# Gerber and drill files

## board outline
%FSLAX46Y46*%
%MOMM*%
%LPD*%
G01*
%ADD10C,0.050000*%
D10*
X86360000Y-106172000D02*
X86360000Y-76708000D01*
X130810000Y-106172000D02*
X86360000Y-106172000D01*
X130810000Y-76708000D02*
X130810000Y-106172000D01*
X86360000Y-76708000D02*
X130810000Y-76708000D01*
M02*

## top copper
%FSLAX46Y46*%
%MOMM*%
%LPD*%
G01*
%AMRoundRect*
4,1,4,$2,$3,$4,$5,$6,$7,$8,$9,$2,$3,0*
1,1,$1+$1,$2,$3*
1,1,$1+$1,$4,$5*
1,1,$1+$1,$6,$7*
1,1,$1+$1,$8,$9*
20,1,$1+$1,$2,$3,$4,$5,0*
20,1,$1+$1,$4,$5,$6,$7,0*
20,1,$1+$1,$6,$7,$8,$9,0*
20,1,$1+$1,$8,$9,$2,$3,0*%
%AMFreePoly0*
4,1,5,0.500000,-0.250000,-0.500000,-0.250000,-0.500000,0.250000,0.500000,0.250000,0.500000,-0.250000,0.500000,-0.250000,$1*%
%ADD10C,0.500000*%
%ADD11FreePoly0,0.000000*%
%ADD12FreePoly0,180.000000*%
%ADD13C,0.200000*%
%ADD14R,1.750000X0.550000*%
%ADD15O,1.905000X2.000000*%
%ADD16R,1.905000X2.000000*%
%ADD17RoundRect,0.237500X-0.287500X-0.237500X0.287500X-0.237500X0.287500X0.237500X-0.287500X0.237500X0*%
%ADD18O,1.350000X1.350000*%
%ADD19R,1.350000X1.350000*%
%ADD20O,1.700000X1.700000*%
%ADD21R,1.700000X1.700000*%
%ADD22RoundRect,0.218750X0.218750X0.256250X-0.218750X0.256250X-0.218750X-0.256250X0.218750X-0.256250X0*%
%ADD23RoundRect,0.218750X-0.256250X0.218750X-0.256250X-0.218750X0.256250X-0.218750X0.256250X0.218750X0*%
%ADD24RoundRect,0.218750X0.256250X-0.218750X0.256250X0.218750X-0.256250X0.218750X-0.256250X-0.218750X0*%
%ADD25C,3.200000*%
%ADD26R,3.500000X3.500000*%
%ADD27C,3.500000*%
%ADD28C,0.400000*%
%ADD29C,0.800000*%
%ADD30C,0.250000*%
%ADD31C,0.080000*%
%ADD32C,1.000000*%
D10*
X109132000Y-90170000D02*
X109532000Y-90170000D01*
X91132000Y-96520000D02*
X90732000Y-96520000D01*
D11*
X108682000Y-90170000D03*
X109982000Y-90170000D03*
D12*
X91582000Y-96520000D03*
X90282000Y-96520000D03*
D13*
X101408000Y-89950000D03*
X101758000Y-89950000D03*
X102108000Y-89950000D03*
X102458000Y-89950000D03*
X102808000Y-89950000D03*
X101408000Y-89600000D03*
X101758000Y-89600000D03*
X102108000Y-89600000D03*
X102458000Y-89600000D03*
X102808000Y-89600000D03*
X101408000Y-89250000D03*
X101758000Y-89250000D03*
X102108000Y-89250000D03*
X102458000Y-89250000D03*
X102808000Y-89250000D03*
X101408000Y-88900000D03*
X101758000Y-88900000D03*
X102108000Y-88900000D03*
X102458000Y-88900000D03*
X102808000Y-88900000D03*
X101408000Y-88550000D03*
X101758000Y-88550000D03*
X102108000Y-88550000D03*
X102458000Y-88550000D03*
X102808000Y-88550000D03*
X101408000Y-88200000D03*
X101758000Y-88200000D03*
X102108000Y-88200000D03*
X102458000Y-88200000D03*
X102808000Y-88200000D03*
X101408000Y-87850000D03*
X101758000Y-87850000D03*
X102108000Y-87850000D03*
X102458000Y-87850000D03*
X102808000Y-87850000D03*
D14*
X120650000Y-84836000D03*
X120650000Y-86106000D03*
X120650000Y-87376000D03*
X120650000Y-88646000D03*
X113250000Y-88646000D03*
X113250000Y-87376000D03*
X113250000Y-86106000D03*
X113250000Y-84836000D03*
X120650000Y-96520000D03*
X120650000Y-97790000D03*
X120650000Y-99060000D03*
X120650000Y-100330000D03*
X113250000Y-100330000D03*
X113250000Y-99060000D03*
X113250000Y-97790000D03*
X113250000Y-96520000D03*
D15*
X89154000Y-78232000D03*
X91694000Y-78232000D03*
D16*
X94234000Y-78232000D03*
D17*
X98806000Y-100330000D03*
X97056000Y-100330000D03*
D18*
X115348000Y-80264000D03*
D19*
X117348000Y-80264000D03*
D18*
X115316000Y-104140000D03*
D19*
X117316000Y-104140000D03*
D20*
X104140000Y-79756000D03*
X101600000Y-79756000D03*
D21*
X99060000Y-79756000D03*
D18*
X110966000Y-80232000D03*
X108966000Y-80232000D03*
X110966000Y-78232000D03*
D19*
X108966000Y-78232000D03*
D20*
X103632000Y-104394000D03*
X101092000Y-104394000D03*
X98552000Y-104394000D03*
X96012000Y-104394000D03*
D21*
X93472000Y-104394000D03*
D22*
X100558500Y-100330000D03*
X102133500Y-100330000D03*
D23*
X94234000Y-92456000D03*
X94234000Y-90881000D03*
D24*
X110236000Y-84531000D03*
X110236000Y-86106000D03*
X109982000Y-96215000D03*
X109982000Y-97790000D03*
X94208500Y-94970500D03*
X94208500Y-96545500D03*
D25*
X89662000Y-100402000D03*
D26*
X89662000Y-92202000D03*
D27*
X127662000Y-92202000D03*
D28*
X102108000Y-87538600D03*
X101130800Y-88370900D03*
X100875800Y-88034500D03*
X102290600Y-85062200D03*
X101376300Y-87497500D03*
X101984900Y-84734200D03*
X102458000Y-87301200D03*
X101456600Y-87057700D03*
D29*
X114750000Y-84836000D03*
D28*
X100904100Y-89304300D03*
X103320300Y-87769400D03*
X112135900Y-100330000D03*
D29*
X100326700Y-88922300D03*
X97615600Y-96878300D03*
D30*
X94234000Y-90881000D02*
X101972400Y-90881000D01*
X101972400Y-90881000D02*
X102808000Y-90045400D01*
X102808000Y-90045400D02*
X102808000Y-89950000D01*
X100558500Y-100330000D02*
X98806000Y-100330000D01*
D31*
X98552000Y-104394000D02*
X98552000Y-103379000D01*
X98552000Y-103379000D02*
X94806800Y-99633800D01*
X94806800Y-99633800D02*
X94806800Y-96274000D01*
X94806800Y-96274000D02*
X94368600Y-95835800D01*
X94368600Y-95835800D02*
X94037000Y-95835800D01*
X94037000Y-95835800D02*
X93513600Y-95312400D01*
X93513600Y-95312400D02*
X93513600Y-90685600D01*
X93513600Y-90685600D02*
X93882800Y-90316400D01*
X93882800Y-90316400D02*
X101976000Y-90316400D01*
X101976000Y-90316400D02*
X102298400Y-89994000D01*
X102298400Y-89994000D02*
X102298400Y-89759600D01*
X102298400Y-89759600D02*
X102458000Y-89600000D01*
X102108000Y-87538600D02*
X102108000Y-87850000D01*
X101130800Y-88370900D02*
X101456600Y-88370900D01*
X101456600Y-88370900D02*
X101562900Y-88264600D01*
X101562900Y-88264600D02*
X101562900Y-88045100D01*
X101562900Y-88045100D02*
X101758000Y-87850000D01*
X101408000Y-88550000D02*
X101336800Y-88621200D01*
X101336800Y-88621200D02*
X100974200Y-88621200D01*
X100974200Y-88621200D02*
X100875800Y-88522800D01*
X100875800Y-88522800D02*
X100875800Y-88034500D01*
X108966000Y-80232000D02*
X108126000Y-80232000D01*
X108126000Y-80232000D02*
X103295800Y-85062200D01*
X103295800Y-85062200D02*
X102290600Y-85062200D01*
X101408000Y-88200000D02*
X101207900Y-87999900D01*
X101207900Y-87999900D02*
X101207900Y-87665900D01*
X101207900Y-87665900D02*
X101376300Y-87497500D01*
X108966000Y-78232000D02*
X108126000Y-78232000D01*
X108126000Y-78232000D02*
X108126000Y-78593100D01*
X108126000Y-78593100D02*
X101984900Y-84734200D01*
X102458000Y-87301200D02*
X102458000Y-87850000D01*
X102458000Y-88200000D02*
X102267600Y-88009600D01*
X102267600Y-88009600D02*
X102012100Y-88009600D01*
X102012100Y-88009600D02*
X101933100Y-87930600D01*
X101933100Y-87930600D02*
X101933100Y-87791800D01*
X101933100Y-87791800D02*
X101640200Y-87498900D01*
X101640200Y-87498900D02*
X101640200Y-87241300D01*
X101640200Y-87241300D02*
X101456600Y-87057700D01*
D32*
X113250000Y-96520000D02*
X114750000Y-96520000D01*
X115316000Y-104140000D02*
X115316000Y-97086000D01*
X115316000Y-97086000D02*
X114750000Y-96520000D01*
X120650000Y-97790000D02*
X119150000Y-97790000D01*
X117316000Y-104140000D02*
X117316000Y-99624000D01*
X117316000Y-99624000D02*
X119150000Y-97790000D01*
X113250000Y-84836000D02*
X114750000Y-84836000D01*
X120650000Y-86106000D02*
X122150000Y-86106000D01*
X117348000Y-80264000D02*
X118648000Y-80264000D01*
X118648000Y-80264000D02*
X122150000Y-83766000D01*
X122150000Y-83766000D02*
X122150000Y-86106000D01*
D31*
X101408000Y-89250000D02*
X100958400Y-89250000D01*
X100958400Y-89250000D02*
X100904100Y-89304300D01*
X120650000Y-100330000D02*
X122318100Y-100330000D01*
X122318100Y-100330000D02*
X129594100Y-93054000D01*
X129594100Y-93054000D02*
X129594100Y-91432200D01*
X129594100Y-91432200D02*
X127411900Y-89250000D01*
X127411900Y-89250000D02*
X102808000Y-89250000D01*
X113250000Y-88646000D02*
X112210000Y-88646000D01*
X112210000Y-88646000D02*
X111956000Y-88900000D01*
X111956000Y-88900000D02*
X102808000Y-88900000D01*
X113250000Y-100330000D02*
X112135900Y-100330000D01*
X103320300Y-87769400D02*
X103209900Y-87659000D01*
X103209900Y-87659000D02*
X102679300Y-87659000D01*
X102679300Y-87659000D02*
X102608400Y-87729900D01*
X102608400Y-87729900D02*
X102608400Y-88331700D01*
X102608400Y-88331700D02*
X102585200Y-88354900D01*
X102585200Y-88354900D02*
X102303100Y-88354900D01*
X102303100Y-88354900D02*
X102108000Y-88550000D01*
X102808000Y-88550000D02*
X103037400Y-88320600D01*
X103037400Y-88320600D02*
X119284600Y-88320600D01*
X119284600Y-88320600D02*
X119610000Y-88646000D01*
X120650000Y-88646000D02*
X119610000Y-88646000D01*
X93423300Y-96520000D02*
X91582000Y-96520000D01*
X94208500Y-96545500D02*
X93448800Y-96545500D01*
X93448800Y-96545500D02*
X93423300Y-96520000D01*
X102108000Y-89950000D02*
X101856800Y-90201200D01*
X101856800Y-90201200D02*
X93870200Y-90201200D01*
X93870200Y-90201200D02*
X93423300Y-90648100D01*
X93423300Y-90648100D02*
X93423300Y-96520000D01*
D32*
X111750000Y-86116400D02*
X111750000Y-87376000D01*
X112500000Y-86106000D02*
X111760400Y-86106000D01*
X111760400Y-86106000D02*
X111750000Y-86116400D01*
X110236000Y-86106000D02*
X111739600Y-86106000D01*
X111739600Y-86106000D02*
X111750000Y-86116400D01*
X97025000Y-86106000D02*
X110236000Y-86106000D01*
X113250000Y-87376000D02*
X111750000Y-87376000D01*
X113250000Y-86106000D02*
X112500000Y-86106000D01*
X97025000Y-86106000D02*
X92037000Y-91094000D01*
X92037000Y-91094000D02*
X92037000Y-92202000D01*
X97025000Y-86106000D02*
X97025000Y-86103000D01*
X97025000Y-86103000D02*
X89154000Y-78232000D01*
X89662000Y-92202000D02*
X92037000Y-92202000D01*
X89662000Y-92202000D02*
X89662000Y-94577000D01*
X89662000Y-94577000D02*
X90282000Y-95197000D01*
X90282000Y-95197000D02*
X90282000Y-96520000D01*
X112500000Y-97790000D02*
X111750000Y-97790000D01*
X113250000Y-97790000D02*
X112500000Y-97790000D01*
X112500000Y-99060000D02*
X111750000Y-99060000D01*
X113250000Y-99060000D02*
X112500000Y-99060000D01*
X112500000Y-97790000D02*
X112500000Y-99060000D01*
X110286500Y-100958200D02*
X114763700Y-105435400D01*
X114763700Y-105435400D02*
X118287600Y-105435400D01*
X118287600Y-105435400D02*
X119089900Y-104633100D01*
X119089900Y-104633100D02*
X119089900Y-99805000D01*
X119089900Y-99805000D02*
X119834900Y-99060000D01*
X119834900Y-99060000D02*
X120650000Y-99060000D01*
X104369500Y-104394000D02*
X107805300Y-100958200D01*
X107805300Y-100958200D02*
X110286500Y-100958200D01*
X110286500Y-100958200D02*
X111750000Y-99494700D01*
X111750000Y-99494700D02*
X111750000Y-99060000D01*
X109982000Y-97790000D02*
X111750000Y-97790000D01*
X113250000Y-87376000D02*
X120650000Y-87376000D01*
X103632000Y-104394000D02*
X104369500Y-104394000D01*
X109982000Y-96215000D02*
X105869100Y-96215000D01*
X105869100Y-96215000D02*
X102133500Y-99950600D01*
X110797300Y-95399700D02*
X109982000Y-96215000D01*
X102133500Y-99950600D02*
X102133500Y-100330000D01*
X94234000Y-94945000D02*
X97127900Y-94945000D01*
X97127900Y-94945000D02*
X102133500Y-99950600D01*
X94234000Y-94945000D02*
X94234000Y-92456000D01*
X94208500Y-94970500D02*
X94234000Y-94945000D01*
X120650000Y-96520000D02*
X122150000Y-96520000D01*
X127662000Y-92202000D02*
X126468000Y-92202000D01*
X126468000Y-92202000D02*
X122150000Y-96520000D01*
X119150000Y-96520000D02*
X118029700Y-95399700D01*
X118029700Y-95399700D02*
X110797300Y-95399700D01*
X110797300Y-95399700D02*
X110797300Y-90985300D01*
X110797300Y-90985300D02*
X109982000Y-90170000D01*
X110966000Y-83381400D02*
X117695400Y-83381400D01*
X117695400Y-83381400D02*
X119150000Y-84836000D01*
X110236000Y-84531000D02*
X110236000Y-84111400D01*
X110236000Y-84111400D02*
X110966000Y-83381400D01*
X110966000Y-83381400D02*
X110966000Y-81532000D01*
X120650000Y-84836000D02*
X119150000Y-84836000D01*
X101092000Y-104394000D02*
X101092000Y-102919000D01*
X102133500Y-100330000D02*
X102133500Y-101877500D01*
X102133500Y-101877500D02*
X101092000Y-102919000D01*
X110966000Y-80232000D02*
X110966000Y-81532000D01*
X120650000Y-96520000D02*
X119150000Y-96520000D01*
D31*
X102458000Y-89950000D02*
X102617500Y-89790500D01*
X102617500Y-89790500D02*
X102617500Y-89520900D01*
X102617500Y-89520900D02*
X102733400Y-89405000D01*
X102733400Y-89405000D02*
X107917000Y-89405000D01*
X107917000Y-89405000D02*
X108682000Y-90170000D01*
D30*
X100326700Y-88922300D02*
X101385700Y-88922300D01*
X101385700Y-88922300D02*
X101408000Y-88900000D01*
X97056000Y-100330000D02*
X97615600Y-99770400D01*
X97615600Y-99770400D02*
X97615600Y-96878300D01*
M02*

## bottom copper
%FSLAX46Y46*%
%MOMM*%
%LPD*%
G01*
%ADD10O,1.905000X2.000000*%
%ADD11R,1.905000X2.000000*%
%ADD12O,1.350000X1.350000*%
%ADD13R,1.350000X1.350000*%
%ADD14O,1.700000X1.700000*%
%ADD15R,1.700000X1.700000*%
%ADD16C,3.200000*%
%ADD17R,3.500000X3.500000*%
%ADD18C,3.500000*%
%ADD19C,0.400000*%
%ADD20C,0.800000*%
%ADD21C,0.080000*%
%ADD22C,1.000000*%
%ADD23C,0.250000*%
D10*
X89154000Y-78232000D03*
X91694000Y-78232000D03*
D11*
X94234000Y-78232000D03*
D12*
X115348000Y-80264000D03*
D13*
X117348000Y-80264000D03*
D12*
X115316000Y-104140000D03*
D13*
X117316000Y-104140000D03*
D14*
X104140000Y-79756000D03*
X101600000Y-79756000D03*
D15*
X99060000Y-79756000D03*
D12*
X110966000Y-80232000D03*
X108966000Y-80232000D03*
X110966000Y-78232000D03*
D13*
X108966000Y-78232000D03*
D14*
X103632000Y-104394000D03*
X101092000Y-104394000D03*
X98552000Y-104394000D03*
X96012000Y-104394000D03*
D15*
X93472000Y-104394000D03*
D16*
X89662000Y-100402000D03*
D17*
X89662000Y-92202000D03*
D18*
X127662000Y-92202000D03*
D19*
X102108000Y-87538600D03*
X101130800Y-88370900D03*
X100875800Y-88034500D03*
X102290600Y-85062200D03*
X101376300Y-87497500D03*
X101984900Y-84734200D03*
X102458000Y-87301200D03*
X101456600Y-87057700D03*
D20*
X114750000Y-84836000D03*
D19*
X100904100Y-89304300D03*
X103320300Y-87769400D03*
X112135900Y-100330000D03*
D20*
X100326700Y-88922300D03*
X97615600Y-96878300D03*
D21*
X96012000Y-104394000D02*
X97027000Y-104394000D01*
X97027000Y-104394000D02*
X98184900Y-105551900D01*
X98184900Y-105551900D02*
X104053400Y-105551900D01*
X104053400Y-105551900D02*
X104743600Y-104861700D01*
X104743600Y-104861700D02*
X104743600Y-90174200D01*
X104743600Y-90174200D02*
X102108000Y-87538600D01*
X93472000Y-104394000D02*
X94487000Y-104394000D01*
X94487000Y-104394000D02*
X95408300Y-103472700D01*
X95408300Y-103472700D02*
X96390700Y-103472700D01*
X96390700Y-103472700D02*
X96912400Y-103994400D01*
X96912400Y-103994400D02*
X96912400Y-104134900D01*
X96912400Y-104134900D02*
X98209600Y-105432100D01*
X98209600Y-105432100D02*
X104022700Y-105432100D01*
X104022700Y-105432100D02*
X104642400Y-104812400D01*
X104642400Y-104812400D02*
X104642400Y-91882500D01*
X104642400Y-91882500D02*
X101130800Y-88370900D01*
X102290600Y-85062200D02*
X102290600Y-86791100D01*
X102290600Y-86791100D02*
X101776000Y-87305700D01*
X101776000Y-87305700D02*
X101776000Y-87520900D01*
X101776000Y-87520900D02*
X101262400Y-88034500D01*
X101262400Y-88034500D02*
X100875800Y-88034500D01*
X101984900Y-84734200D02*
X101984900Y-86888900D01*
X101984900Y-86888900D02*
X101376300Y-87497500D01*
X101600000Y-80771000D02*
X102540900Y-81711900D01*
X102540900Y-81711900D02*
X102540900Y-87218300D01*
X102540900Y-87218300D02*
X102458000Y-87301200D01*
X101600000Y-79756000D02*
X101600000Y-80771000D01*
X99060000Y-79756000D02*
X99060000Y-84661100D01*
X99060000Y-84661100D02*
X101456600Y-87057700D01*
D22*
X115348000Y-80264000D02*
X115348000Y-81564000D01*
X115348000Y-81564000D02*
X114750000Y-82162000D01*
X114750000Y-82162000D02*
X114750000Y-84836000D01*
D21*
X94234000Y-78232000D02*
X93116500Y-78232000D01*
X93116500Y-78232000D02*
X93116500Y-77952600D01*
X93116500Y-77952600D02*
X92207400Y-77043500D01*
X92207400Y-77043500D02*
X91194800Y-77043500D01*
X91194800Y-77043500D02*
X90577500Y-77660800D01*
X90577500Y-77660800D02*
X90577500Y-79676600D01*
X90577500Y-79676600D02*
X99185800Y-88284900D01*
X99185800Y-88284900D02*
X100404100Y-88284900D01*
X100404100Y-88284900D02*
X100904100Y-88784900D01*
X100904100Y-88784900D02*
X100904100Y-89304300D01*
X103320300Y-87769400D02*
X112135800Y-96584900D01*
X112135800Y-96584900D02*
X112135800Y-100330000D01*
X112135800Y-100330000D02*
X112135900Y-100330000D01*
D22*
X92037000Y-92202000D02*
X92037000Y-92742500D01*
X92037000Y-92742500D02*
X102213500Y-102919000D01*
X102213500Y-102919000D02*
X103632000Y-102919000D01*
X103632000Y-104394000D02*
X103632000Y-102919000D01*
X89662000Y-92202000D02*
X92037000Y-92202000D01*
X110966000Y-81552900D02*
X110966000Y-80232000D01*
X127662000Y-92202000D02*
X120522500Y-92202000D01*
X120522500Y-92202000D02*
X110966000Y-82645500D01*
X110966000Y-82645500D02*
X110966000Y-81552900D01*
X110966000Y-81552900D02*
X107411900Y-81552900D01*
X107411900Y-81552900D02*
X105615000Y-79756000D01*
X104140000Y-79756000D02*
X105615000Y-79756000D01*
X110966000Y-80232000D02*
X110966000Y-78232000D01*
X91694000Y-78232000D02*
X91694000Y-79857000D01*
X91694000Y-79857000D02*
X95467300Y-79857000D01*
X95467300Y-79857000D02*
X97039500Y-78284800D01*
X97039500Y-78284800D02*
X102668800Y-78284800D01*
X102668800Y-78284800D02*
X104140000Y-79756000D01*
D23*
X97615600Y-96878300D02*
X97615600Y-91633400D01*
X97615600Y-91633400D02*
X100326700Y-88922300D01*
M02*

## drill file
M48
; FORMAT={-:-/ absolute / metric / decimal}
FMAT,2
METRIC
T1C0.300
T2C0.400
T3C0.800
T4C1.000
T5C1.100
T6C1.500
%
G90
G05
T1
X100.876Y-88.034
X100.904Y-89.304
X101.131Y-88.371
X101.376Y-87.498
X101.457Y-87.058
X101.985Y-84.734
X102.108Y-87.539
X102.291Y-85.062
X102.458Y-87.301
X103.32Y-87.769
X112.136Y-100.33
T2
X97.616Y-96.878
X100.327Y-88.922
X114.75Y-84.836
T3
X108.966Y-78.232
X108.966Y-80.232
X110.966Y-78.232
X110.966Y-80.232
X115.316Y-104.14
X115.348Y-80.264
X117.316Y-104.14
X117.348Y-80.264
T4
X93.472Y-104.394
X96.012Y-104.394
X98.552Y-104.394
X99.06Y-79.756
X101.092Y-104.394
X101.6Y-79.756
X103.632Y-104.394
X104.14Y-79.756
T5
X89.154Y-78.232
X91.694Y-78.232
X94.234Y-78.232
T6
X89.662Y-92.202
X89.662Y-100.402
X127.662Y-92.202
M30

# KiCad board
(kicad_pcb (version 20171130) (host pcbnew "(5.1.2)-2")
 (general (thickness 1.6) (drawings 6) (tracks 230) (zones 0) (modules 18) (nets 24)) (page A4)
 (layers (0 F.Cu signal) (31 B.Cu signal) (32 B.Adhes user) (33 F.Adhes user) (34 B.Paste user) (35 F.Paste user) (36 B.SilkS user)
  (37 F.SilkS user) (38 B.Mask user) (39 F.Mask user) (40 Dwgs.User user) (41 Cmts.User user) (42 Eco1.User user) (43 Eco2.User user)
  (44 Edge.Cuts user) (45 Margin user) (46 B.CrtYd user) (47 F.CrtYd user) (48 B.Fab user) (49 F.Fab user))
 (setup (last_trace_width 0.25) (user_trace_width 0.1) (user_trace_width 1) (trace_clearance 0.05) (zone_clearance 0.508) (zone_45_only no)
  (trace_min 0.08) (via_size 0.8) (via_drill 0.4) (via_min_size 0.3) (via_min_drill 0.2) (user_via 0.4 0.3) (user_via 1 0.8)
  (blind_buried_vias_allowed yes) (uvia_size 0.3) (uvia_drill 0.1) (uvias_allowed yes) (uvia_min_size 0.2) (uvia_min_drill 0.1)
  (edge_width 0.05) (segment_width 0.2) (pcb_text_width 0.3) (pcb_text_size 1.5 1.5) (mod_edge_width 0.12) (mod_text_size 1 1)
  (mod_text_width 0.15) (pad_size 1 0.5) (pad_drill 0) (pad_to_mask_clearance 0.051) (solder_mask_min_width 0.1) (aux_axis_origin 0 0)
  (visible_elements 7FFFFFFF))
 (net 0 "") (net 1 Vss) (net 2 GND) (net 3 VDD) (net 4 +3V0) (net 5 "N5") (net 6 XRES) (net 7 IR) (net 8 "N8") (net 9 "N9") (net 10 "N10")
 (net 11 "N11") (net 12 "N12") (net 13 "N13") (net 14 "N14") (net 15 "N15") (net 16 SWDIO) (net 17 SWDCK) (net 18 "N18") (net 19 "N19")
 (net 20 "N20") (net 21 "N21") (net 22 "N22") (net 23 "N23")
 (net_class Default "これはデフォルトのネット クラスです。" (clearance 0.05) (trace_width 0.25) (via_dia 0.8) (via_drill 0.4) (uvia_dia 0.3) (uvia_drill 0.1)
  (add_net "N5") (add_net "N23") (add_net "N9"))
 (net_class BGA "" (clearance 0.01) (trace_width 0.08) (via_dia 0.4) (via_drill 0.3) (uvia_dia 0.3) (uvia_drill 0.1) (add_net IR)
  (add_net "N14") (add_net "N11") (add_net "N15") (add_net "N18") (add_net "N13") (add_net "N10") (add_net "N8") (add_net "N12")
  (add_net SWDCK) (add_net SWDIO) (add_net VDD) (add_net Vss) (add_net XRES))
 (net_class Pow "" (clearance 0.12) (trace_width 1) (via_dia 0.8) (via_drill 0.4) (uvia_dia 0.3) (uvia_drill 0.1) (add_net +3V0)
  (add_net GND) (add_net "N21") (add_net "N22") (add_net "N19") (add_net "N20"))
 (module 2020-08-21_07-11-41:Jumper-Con (layer F.Cu) (at 109.332 90.17)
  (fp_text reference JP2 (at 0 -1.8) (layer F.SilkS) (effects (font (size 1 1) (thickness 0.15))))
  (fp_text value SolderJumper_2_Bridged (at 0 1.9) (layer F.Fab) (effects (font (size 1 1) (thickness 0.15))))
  (fp_line (start -0.2 0) (end 0.2 0) (layer F.Cu) (width 0.5))
  (pad 1 smd custom (at -0.65 0) (size 1 0.5) (layers F.Cu F.Adhes F.Mask) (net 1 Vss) (zone_connect 2)
   (options (clearance outline) (anchor rect)) (primitives))
  (pad 2 smd custom (at 0.65 0) (size 1 0.5) (layers F.Cu F.Adhes F.Mask) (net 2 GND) (zone_connect 2)
   (options (clearance outline) (anchor rect)) (primitives)))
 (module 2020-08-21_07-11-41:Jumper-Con (layer F.Cu) (at 90.932 96.52 180)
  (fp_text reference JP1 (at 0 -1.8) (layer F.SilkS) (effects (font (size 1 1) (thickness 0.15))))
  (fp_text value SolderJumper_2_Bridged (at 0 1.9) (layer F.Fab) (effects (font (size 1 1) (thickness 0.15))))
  (fp_line (start -0.2 0) (end 0.2 0) (layer F.Cu) (width 0.5))
  (pad 1 smd custom (at -0.65 0 180) (size 1 0.5) (layers F.Cu F.Adhes F.Mask) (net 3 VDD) (zone_connect 2)
   (options (clearance outline) (anchor rect)) (primitives))
  (pad 2 smd custom (at 0.65 0 180) (size 1 0.5) (layers F.Cu F.Adhes F.Mask) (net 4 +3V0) (zone_connect 2)
   (options (clearance outline) (anchor rect)) (primitives)))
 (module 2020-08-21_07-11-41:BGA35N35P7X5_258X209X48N (layer F.Cu) (at 102.108 88.9 270) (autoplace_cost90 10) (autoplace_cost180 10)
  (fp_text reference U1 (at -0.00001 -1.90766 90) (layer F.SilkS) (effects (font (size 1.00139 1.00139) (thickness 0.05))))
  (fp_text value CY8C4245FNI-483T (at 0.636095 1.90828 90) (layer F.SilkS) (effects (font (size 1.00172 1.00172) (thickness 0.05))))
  (pad E7 smd circle (at 1.05 0.7 90) (size 0.2 0.2) (layers F.Cu F.Paste F.Mask))
  (pad D7 smd circle (at 1.05 0.35 270) (size 0.2 0.2) (layers F.Cu F.Paste F.Mask))
  (pad C7 smd circle (at 1.05 0 270) (size 0.2 0.2) (layers F.Cu F.Paste F.Mask) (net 3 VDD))
  (pad B7 smd circle (at 1.05 -0.35 270) (size 0.2 0.2) (layers F.Cu F.Paste F.Mask) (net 1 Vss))
  (pad A7 smd circle (at 1.05 -0.7 270) (size 0.2 0.2) (layers F.Cu F.Paste F.Mask) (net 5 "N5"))
  (pad E6 smd circle (at 0.7 0.7 270) (size 0.2 0.2) (layers F.Cu F.Paste F.Mask))
  (pad D6 smd circle (at 0.7 0.35 270) (size 0.2 0.2) (layers F.Cu F.Paste F.Mask))
  (pad C6 smd circle (at 0.7 0 270) (size 0.2 0.2) (layers F.Cu F.Paste F.Mask))
  (pad B6 smd circle (at 0.7 -0.35 270) (size 0.2 0.2) (layers F.Cu F.Paste F.Mask) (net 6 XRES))
  (pad A6 smd circle (at 0.7 -0.7 270) (size 0.2 0.2) (layers F.Cu F.Paste F.Mask))
  (pad E5 smd circle (at 0.35 0.7 270) (size 0.2 0.2) (layers F.Cu F.Paste F.Mask) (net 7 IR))
  (pad D5 smd circle (at 0.35 0.35 270) (size 0.2 0.2) (layers F.Cu F.Paste F.Mask))
  (pad C5 smd circle (at 0.35 0 270) (size 0.2 0.2) (layers F.Cu F.Paste F.Mask))
  (pad B5 smd circle (at 0.35 -0.35 270) (size 0.2 0.2) (layers F.Cu F.Paste F.Mask))
  (pad A5 smd circle (at 0.35 -0.7 270) (size 0.2 0.2) (layers F.Cu F.Paste F.Mask) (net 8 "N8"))
  (pad E4 smd circle (at 0 0.7 270) (size 0.2 0.2) (layers F.Cu F.Paste F.Mask) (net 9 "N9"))
  (pad D4 smd circle (at 0 0.35 270) (size 0.2 0.2) (layers F.Cu F.Paste F.Mask))
  (pad C4 smd circle (at 0 0 270) (size 0.2 0.2) (layers F.Cu F.Paste F.Mask))
  (pad B4 smd circle (at 0 -0.35 270) (size 0.2 0.2) (layers F.Cu F.Paste F.Mask))
  (pad A4 smd circle (at 0 -0.7 270) (size 0.2 0.2) (layers F.Cu F.Paste F.Mask) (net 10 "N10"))
  (pad E3 smd circle (at -0.35 0.7 270) (size 0.2 0.2) (layers F.Cu F.Paste F.Mask) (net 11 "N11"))
  (pad D3 smd circle (at -0.35 0.35 270) (size 0.2 0.2) (layers F.Cu F.Paste F.Mask))
  (pad C3 smd circle (at -0.35 0 270) (size 0.2 0.2) (layers F.Cu F.Paste F.Mask) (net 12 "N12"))
  (pad B3 smd circle (at -0.35 -0.35 270) (size 0.2 0.2) (layers F.Cu F.Paste F.Mask))
  (pad A3 smd circle (at -0.35 -0.7 270) (size 0.2 0.2) (layers F.Cu F.Paste F.Mask) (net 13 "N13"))
  (pad E2 smd circle (at -0.7 0.7 270) (size 0.2 0.2) (layers F.Cu F.Paste F.Mask) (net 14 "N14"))
  (pad D2 smd circle (at -0.7 0.35 270) (size 0.2 0.2) (layers F.Cu F.Paste F.Mask))
  (pad C2 smd circle (at -0.7 0 270) (size 0.2 0.2) (layers F.Cu F.Paste F.Mask))
  (pad B2 smd circle (at -0.7 -0.35 270) (size 0.2 0.2) (layers F.Cu F.Paste F.Mask) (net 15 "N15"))
  (pad A2 smd circle (at -0.7 -0.7 270) (size 0.2 0.2) (layers F.Cu F.Paste F.Mask))
  (pad E1 smd circle (at -1.05 0.7 270) (size 0.2 0.2) (layers F.Cu F.Paste F.Mask))
  (pad D1 smd circle (at -1.05 0.35 270) (size 0.2 0.2) (layers F.Cu F.Paste F.Mask) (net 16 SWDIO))
  (pad C1 smd circle (at -1.05 0 270) (size 0.2 0.2) (layers F.Cu F.Paste F.Mask) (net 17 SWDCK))
  (pad B1 smd circle (at -1.05 -0.35 270) (size 0.2 0.2) (layers F.Cu F.Paste F.Mask) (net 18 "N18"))
  (pad A1 smd circle (at -1.05 -0.7) (size 0.2 0.2) (layers F.Cu F.Paste F.Mask)))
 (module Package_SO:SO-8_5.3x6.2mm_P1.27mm (layer F.Cu) (at 116.95 86.741)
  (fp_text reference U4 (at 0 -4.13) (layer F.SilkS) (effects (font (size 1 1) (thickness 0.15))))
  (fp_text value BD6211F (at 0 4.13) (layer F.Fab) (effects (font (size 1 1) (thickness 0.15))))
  (pad 8 smd rect (at 3.7 -1.905) (size 1.75 0.55) (layers F.Cu F.Paste F.Mask) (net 2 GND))
  (pad 7 smd rect (at 3.7 -0.635) (size 1.75 0.55) (layers F.Cu F.Paste F.Mask) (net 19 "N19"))
  (pad 6 smd rect (at 3.7 0.635) (size 1.75 0.55) (layers F.Cu F.Paste F.Mask) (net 4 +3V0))
  (pad 5 smd rect (at 3.7 1.905) (size 1.75 0.55) (layers F.Cu F.Paste F.Mask) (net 13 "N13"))
  (pad 4 smd rect (at -3.7 1.905) (size 1.75 0.55) (layers F.Cu F.Paste F.Mask) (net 10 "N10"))
  (pad 3 smd rect (at -3.7 0.635) (size 1.75 0.55) (layers F.Cu F.Paste F.Mask) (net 4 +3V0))
  (pad 2 smd rect (at -3.7 -0.635) (size 1.75 0.55) (layers F.Cu F.Paste F.Mask) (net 4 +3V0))
  (pad 1 smd rect (at -3.7 -1.905) (size 1.75 0.55) (layers F.Cu F.Paste F.Mask) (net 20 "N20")))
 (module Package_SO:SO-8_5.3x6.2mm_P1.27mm (layer F.Cu) (at 116.95 98.425)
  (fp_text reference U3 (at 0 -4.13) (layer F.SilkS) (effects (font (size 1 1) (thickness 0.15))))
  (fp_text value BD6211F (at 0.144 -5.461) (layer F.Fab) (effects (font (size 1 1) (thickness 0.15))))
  (pad 8 smd rect (at 3.7 -1.905) (size 1.75 0.55) (layers F.Cu F.Paste F.Mask) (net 2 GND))
  (pad 7 smd rect (at 3.7 -0.635) (size 1.75 0.55) (layers F.Cu F.Paste F.Mask) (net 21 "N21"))
  (pad 6 smd rect (at 3.7 0.635) (size 1.75 0.55) (layers F.Cu F.Paste F.Mask) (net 4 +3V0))
  (pad 5 smd rect (at 3.7 1.905) (size 1.75 0.55) (layers F.Cu F.Paste F.Mask) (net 8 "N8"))
  (pad 4 smd rect (at -3.7 1.905) (size 1.75 0.55) (layers F.Cu F.Paste F.Mask) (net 12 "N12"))
  (pad 3 smd rect (at -3.7 0.635) (size 1.75 0.55) (layers F.Cu F.Paste F.Mask) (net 4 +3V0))
  (pad 2 smd rect (at -3.7 -0.635) (size 1.75 0.55) (layers F.Cu F.Paste F.Mask) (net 4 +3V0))
  (pad 1 smd rect (at -3.7 -1.905) (size 1.75 0.55) (layers F.Cu F.Paste F.Mask) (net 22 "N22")))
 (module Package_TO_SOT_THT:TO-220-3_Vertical (layer F.Cu) (at 94.234 78.232 180)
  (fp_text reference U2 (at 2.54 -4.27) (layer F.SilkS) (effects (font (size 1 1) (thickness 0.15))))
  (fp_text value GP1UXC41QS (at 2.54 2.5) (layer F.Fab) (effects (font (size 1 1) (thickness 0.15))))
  (pad 3 thru_hole oval (at 5.08 0 180) (size 1.905 2) (drill 1.1) (layers *.Cu *.Mask) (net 4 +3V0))
  (pad 2 thru_hole oval (at 2.54 0 180) (size 1.905 2) (drill 1.1) (layers *.Cu *.Mask) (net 2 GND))
  (pad 1 thru_hole rect (at 0 0 180) (size 1.905 2) (drill 1.1) (layers *.Cu *.Mask) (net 7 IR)))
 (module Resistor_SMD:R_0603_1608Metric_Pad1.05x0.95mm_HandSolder (layer F.Cu) (at 97.931 100.33)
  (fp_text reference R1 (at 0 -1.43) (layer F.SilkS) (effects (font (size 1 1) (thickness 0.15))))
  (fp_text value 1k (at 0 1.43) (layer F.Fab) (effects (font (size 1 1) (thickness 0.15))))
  (pad 2 smd roundrect (at 0.875 0) (size 1.05 0.95) (layers F.Cu F.Paste F.Mask) (roundrect_rratio 0.25) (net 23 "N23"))
  (pad 1 smd roundrect (at -0.875 0) (size 1.05 0.95) (layers F.Cu F.Paste F.Mask) (roundrect_rratio 0.25) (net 9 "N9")))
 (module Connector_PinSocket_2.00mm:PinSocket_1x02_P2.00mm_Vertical (layer F.Cu) (at 117.348 80.264 270)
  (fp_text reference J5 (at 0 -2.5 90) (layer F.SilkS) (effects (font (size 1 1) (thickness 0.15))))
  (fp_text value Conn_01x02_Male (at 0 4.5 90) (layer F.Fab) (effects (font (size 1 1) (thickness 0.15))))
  (pad 2 thru_hole oval (at 0 2 270) (size 1.35 1.35) (drill 0.8) (layers *.Cu *.Mask) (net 20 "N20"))
  (pad 1 thru_hole rect (at 0 0 270) (size 1.35 1.35) (drill 0.8) (layers *.Cu *.Mask) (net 19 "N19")))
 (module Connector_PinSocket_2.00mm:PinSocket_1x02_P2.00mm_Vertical (layer F.Cu) (at 117.316 104.14 270)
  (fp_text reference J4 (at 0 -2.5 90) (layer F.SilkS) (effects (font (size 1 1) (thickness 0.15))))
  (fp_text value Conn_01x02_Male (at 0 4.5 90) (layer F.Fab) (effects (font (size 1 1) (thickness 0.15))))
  (pad 2 thru_hole oval (at 0 2 270) (size 1.35 1.35) (drill 0.8) (layers *.Cu *.Mask) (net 22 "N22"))
  (pad 1 thru_hole rect (at 0 0 270) (size 1.35 1.35) (drill 0.8) (layers *.Cu *.Mask) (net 21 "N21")))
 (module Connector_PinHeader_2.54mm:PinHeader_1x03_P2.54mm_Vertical (layer F.Cu) (at 99.06 79.756 90)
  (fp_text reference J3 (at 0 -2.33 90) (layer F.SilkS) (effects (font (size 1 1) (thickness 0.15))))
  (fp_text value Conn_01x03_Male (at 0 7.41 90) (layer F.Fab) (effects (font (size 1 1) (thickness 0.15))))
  (pad 3 thru_hole oval (at 0 5.08 90) (size 1.7 1.7) (drill 1) (layers *.Cu *.Mask) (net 2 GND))
  (pad 2 thru_hole oval (at 0 2.54 90) (size 1.7 1.7) (drill 1) (layers *.Cu *.Mask) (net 18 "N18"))
  (pad 1 thru_hole rect (at 0 0 90) (size 1.7 1.7) (drill 1) (layers *.Cu *.Mask) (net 15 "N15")))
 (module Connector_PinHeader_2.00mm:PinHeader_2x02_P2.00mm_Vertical (layer F.Cu) (at 108.966 78.232)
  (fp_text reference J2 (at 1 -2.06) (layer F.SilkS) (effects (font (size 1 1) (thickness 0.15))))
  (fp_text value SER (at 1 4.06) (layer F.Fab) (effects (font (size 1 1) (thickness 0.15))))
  (pad 4 thru_hole oval (at 2 2) (size 1.35 1.35) (drill 0.8) (layers *.Cu *.Mask) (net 2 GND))
  (pad 3 thru_hole oval (at 0 2) (size 1.35 1.35) (drill 0.8) (layers *.Cu *.Mask) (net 11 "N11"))
  (pad 2 thru_hole oval (at 2 0) (size 1.35 1.35) (drill 0.8) (layers *.Cu *.Mask) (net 2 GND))
  (pad 1 thru_hole rect (at 0 0) (size 1.35 1.35) (drill 0.8) (layers *.Cu *.Mask) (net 14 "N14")))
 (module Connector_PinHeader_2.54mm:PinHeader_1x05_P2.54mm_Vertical (layer F.Cu) (at 93.472 104.394 90)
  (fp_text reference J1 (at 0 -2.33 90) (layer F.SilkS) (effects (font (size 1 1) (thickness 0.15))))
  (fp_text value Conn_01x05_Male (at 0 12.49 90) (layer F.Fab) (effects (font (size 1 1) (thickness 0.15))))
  (pad 5 thru_hole oval (at 0 10.16 90) (size 1.7 1.7) (drill 1) (layers *.Cu *.Mask) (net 4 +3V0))
  (pad 4 thru_hole oval (at 0 7.62 90) (size 1.7 1.7) (drill 1) (layers *.Cu *.Mask) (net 2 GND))
  (pad 3 thru_hole oval (at 0 5.08 90) (size 1.7 1.7) (drill 1) (layers *.Cu *.Mask) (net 6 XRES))
  (pad 2 thru_hole oval (at 0 2.54 90) (size 1.7 1.7) (drill 1) (layers *.Cu *.Mask) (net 17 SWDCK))
  (pad 1 thru_hole rect (at 0 0 90) (size 1.7 1.7) (drill 1) (layers *.Cu *.Mask) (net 16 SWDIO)))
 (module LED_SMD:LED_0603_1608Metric (layer F.Cu) (at 101.346 100.33 180)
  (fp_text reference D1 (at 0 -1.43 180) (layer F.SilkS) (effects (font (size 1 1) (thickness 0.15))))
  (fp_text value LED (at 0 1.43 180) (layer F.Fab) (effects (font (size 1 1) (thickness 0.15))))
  (pad 2 smd roundrect (at 0.7875 0 180) (size 0.875 0.95) (layers F.Cu F.Paste F.Mask) (roundrect_rratio 0.25) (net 23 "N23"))
  (pad 1 smd roundrect (at -0.7875 0 180) (size 0.875 0.95) (layers F.Cu F.Paste F.Mask) (roundrect_rratio 0.25) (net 2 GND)))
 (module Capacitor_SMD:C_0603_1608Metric (layer F.Cu) (at 94.234 91.6685 270)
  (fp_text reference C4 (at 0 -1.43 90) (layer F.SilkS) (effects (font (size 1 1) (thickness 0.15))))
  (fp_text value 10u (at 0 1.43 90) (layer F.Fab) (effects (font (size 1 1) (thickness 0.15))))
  (pad 2 smd roundrect (at 0.7875 0 270) (size 0.875 0.95) (layers F.Cu F.Paste F.Mask) (roundrect_rratio 0.25) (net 2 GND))
  (pad 1 smd roundrect (at -0.7875 0 270) (size 0.875 0.95) (layers F.Cu F.Paste F.Mask) (roundrect_rratio 0.25) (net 5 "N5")))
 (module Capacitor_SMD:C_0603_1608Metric (layer F.Cu) (at 110.236 85.3185 90)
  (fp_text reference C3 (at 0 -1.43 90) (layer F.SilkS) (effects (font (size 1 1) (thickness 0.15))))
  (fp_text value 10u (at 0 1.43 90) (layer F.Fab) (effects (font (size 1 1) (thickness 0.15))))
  (pad 2 smd roundrect (at 0.7875 0 90) (size 0.875 0.95) (layers F.Cu F.Paste F.Mask) (roundrect_rratio 0.25) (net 2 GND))
  (pad 1 smd roundrect (at -0.7875 0 90) (size 0.875 0.95) (layers F.Cu F.Paste F.Mask) (roundrect_rratio 0.25) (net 4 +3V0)))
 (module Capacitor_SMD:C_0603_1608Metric (layer F.Cu) (at 109.982 97.0025 90)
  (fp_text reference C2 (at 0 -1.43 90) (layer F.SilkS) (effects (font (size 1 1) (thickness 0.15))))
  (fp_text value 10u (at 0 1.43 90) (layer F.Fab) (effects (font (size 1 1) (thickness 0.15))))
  (pad 2 smd roundrect (at 0.7875 0 90) (size 0.875 0.95) (layers F.Cu F.Paste F.Mask) (roundrect_rratio 0.25) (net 2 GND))
  (pad 1 smd roundrect (at -0.7875 0 90) (size 0.875 0.95) (layers F.Cu F.Paste F.Mask) (roundrect_rratio 0.25) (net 4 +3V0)))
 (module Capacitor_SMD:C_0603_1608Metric (layer F.Cu) (at 94.2085 95.758 90)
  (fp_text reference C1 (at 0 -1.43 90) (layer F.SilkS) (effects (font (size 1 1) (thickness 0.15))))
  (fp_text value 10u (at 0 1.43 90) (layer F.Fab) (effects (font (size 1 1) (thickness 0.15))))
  (pad 2 smd roundrect (at 0.7875 0 90) (size 0.875 0.95) (layers F.Cu F.Paste F.Mask) (roundrect_rratio 0.25) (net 2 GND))
  (pad 1 smd roundrect (at -0.7875 0 90) (size 0.875 0.95) (layers F.Cu F.Paste F.Mask) (roundrect_rratio 0.25) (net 3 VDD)))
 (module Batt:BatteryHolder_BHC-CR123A (layer B.Cu) (at 89.662 92.202)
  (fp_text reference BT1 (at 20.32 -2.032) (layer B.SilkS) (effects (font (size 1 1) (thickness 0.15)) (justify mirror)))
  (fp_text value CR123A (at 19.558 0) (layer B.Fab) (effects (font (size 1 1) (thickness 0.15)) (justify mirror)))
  (pad "" thru_hole circle (at 0 8.2) (size 3.2 3.2) (drill 1.5) (layers *.Cu *.Mask))
  (pad 1 thru_hole rect (at 0 0) (size 3.5 3.5) (drill 1.5) (layers *.Cu *.Mask) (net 4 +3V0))
  (pad 2 thru_hole circle (at 38 0) (size 3.5 3.5) (drill 1.5) (layers *.Cu *.Mask) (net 2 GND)))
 (gr_line (start 86.36 106.172) (end 86.36 76.708) (layer Edge.Cuts) (width 0.05))
 (gr_line (start 130.81 106.172) (end 86.36 106.172) (layer Edge.Cuts) (width 0.05))
 (gr_line (start 130.81 76.708) (end 130.81 106.172) (layer Edge.Cuts) (width 0.05))
 (gr_line (start 86.36 76.708) (end 130.81 76.708) (layer Edge.Cuts) (width 0.05))
 (segment (start 94.234 90.881) (end 101.9724 90.881) (width 0.25) (layer F.Cu) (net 5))
 (segment (start 101.9724 90.881) (end 102.808 90.0454) (width 0.25) (layer F.Cu) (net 5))
 (segment (start 102.808 90.0454) (end 102.808 89.95) (width 0.25) (layer F.Cu) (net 5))
 (segment (start 100.5585 100.33) (end 98.806 100.33) (width 0.25) (layer F.Cu) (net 23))
 (segment (start 98.552 104.394) (end 98.552 103.379) (width 0.08) (layer F.Cu) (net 6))
 (segment (start 98.552 103.379) (end 94.8068 99.6338) (width 0.08) (layer F.Cu) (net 6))
 (segment (start 94.8068 99.6338) (end 94.8068 96.274) (width 0.08) (layer F.Cu) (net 6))
 (segment (start 94.8068 96.274) (end 94.3686 95.8358) (width 0.08) (layer F.Cu) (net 6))
 (segment (start 94.3686 95.8358) (end 94.037 95.8358) (width 0.08) (layer F.Cu) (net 6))
 (segment (start 94.037 95.8358) (end 93.5136 95.3124) (width 0.08) (layer F.Cu) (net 6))
 (segment (start 93.5136 95.3124) (end 93.5136 90.6856) (width 0.08) (layer F.Cu) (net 6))
 (segment (start 93.5136 90.6856) (end 93.8828 90.3164) (width 0.08) (layer F.Cu) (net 6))
 (segment (start 93.8828 90.3164) (end 101.976 90.3164) (width 0.08) (layer F.Cu) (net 6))
 (segment (start 101.976 90.3164) (end 102.2984 89.994) (width 0.08) (layer F.Cu) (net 6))
 (segment (start 102.2984 89.994) (end 102.2984 89.7596) (width 0.08) (layer F.Cu) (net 6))
 (segment (start 102.2984 89.7596) (end 102.458 89.6) (width 0.08) (layer F.Cu) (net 6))
 (segment (start 96.012 104.394) (end 97.027 104.394) (width 0.08) (layer B.Cu) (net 17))
 (segment (start 102.108 87.5386) (end 102.108 87.85) (width 0.08) (layer F.Cu) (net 17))
 (segment (start 97.027 104.394) (end 98.1849 105.5519) (width 0.08) (layer B.Cu) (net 17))
 (segment (start 98.1849 105.5519) (end 104.0534 105.5519) (width 0.08) (layer B.Cu) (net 17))
 (segment (start 104.0534 105.5519) (end 104.7436 104.8617) (width 0.08) (layer B.Cu) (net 17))
 (segment (start 104.7436 104.8617) (end 104.7436 90.1742) (width 0.08) (layer B.Cu) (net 17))
 (segment (start 104.7436 90.1742) (end 102.108 87.5386) (width 0.08) (layer B.Cu) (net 17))
 (via (at 102.108 87.5386) (size 0.4) (drill 0.3) (layers F.Cu B.Cu) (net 17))
 (segment (start 93.472 104.394) (end 94.487 104.394) (width 0.08) (layer B.Cu) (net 16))
 (segment (start 101.1308 88.3709) (end 101.4566 88.3709) (width 0.08) (layer F.Cu) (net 16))
 (segment (start 101.4566 88.3709) (end 101.5629 88.2646) (width 0.08) (layer F.Cu) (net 16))
 (segment (start 101.5629 88.2646) (end 101.5629 88.0451) (width 0.08) (layer F.Cu) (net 16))
 (segment (start 101.5629 88.0451) (end 101.758 87.85) (width 0.08) (layer F.Cu) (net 16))
 (segment (start 94.487 104.394) (end 95.4083 103.4727) (width 0.08) (layer B.Cu) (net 16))
 (segment (start 95.4083 103.4727) (end 96.3907 103.4727) (width 0.08) (layer B.Cu) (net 16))
 (segment (start 96.3907 103.4727) (end 96.9124 103.9944) (width 0.08) (layer B.Cu) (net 16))
 (segment (start 96.9124 103.9944) (end 96.9124 104.1349) (width 0.08) (layer B.Cu) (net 16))
 (segment (start 96.9124 104.1349) (end 98.2096 105.4321) (width 0.08) (layer B.Cu) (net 16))
 (segment (start 98.2096 105.4321) (end 104.0227 105.4321) (width 0.08) (layer B.Cu) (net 16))
 (segment (start 104.0227 105.4321) (end 104.6424 104.8124) (width 0.08) (layer B.Cu) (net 16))
 (segment (start 104.6424 104.8124) (end 104.6424 91.8825) (width 0.08) (layer B.Cu) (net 16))
 (segment (start 104.6424 91.8825) (end 101.1308 88.3709) (width 0.08) (layer B.Cu) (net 16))
 (via (at 101.1308 88.3709) (size 0.4) (drill 0.3) (layers F.Cu B.Cu) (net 16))
 (segment (start 101.408 88.55) (end 101.3368 88.6212) (width 0.08) (layer F.Cu) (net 11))
 (segment (start 101.3368 88.6212) (end 100.9742 88.6212) (width 0.08) (layer F.Cu) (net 11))
 (segment (start 100.9742 88.6212) (end 100.8758 88.5228) (width 0.08) (layer F.Cu) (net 11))
 (segment (start 100.8758 88.5228) (end 100.8758 88.0345) (width 0.08) (layer F.Cu) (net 11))
 (segment (start 102.2906 85.0622) (end 102.2906 86.7911) (width 0.08) (layer B.Cu) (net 11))
 (segment (start 102.2906 86.7911) (end 101.776 87.3057) (width 0.08) (layer B.Cu) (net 11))
 (segment (start 101.776 87.3057) (end 101.776 87.5209) (width 0.08) (layer B.Cu) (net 11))
 (segment (start 101.776 87.5209) (end 101.2624 88.0345) (width 0.08) (layer B.Cu) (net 11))
 (segment (start 101.2624 88.0345) (end 100.8758 88.0345) (width 0.08) (layer B.Cu) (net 11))
 (segment (start 108.966 80.232) (end 108.126 80.232) (width 0.08) (layer F.Cu) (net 11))
 (segment (start 108.126 80.232) (end 103.2958 85.0622) (width 0.08) (layer F.Cu) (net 11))
 (segment (start 103.2958 85.0622) (end 102.2906 85.0622) (width 0.08) (layer F.Cu) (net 11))
 (via (at 100.8758 88.0345) (size 0.4) (drill 0.3) (layers F.Cu B.Cu) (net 11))
 (via (at 102.2906 85.0622) (size 0.4) (drill 0.3) (layers F.Cu B.Cu) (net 11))
 (segment (start 101.408 88.2) (end 101.2079 87.9999) (width 0.08) (layer F.Cu) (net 14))
 (segment (start 101.2079 87.9999) (end 101.2079 87.6659) (width 0.08) (layer F.Cu) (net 14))
 (segment (start 101.2079 87.6659) (end 101.3763 87.4975) (width 0.08) (layer F.Cu) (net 14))
 (segment (start 101.9849 84.7342) (end 101.9849 86.8889) (width 0.08) (layer B.Cu) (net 14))
 (segment (start 101.9849 86.8889) (end 101.3763 87.4975) (width 0.08) (layer B.Cu) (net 14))
 (segment (start 108.966 78.232) (end 108.126 78.232) (width 0.08) (layer F.Cu) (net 14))
 (segment (start 108.126 78.232) (end 108.126 78.5931) (width 0.08) (layer F.Cu) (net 14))
 (segment (start 108.126 78.5931) (end 101.9849 84.7342) (width 0.08) (layer F.Cu) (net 14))
 (via (at 101.3763 87.4975) (size 0.4) (drill 0.3) (layers F.Cu B.Cu) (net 14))
 (via (at 101.9849 84.7342) (size 0.4) (drill 0.3) (layers F.Cu B.Cu) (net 14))
 (segment (start 102.458 87.3012) (end 102.458 87.85) (width 0.08) (layer F.Cu) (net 18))
 (segment (start 101.6 80.771) (end 102.5409 81.7119) (width 0.08) (layer B.Cu) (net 18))
 (segment (start 102.5409 81.7119) (end 102.5409 87.2183) (width 0.08) (layer B.Cu) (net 18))
 (segment (start 102.5409 87.2183) (end 102.458 87.3012) (width 0.08) (layer B.Cu) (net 18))
 (segment (start 101.6 79.756) (end 101.6 80.771) (width 0.08) (layer B.Cu) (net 18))
 (via (at 102.458 87.3012) (size 0.4) (drill 0.3) (layers F.Cu B.Cu) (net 18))
 (segment (start 102.458 88.2) (end 102.2676 88.0096) (width 0.08) (layer F.Cu) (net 15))
 (segment (start 102.2676 88.0096) (end 102.0121 88.0096) (width 0.08) (layer F.Cu) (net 15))
 (segment (start 102.0121 88.0096) (end 101.9331 87.9306) (width 0.08) (layer F.Cu) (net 15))
 (segment (start 101.9331 87.9306) (end 101.9331 87.7918) (width 0.08) (layer F.Cu) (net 15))
 (segment (start 101.9331 87.7918) (end 101.6402 87.4989) (width 0.08) (layer F.Cu) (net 15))
 (segment (start 101.6402 87.4989) (end 101.6402 87.2413) (width 0.08) (layer F.Cu) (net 15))
 (segment (start 101.6402 87.2413) (end 101.4566 87.0577) (width 0.08) (layer F.Cu) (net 15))
 (segment (start 99.06 79.756) (end 99.06 84.6611) (width 0.08) (layer B.Cu) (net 15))
 (segment (start 99.06 84.6611) (end 101.4566 87.0577) (width 0.08) (layer B.Cu) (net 15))
 (via (at 101.4566 87.0577) (size 0.4) (drill 0.3) (layers F.Cu B.Cu) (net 15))
 (segment (start 113.25 96.52) (end 114.75 96.52) (width 1) (layer F.Cu) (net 22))
 (segment (start 115.316 104.14) (end 115.316 97.086) (width 1) (layer F.Cu) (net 22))
 (segment (start 115.316 97.086) (end 114.75 96.52) (width 1) (layer F.Cu) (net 22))
 (segment (start 120.65 97.79) (end 119.15 97.79) (width 1) (layer F.Cu) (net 21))
 (segment (start 117.316 104.14) (end 117.316 99.624) (width 1) (layer F.Cu) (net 21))
 (segment (start 117.316 99.624) (end 119.15 97.79) (width 1) (layer F.Cu) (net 21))
 (segment (start 115.348 80.264) (end 115.348 81.564) (width 1) (layer B.Cu) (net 20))
 (segment (start 115.348 81.564) (end 114.75 82.162) (width 1) (layer B.Cu) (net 20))
 (segment (start 114.75 82.162) (end 114.75 84.836) (width 1) (layer B.Cu) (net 20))
 (segment (start 113.25 84.836) (end 114.75 84.836) (width 1) (layer F.Cu) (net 20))
 (via (at 114.75 84.836) (size 0.8) (layers F.Cu B.Cu) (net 20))
 (segment (start 120.65 86.106) (end 122.15 86.106) (width 1) (layer F.Cu) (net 19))
 (segment (start 117.348 80.264) (end 118.648 80.264) (width 1) (layer F.Cu) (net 19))
 (segment (start 118.648 80.264) (end 122.15 83.766) (width 1) (layer F.Cu) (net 19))
 (segment (start 122.15 83.766) (end 122.15 86.106) (width 1) (layer F.Cu) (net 19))
 (segment (start 94.234 78.232) (end 93.1165 78.232) (width 0.08) (layer B.Cu) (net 7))
 (segment (start 101.408 89.25) (end 100.9584 89.25) (width 0.08) (layer F.Cu) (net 7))
 (segment (start 100.9584 89.25) (end 100.9041 89.3043) (width 0.08) (layer F.Cu) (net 7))
 (segment (start 93.1165 78.232) (end 93.1165 77.9526) (width 0.08) (layer B.Cu) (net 7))
 (segment (start 93.1165 77.9526) (end 92.2074 77.0435) (width 0.08) (layer B.Cu) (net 7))
 (segment (start 92.2074 77.0435) (end 91.1948 77.0435) (width 0.08) (layer B.Cu) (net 7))
 (segment (start 91.1948 77.0435) (end 90.5775 77.6608) (width 0.08) (layer B.Cu) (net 7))
 (segment (start 90.5775 77.6608) (end 90.5775 79.6766) (width 0.08) (layer B.Cu) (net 7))
 (segment (start 90.5775 79.6766) (end 99.1858 88.2849) (width 0.08) (layer B.Cu) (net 7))
 (segment (start 99.1858 88.2849) (end 100.4041 88.2849) (width 0.08) (layer B.Cu) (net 7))
 (segment (start 100.4041 88.2849) (end 100.9041 88.7849) (width 0.08) (layer B.Cu) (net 7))
 (segment (start 100.9041 88.7849) (end 100.9041 89.3043) (width 0.08) (layer B.Cu) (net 7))
 (via (at 100.9041 89.3043) (size 0.4) (drill 0.3) (layers F.Cu B.Cu) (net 7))
 (segment (start 120.65 100.33) (end 122.3181 100.33) (width 0.08) (layer F.Cu) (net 8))
 (segment (start 122.3181 100.33) (end 129.5941 93.054) (width 0.08) (layer F.Cu) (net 8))
 (segment (start 129.5941 93.054) (end 129.5941 91.4322) (width 0.08) (layer F.Cu) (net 8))
 (segment (start 129.5941 91.4322) (end 127.4119 89.25) (width 0.08) (layer F.Cu) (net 8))
 (segment (start 127.4119 89.25) (end 102.808 89.25) (width 0.08) (layer F.Cu) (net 8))
 (segment (start 113.25 88.646) (end 112.21 88.646) (width 0.08) (layer F.Cu) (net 10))
 (segment (start 112.21 88.646) (end 111.956 88.9) (width 0.08) (layer F.Cu) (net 10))
 (segment (start 111.956 88.9) (end 102.808 88.9) (width 0.08) (layer F.Cu) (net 10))
 (segment (start 113.25 100.33) (end 112.1359 100.33) (width 0.08) (layer F.Cu) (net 12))
 (segment (start 103.3203 87.7694) (end 112.1358 96.5849) (width 0.08) (layer B.Cu) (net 12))
 (segment (start 112.1358 96.5849) (end 112.1358 100.33) (width 0.08) (layer B.Cu) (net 12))
 (segment (start 112.1358 100.33) (end 112.1359 100.33) (width 0.08) (layer B.Cu) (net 12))
 (segment (start 103.3203 87.7694) (end 103.2099 87.659) (width 0.08) (layer F.Cu) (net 12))
 (segment (start 103.2099 87.659) (end 102.6793 87.659) (width 0.08) (layer F.Cu) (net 12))
 (segment (start 102.6793 87.659) (end 102.6084 87.7299) (width 0.08) (layer F.Cu) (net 12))
 (segment (start 102.6084 87.7299) (end 102.6084 88.3317) (width 0.08) (layer F.Cu) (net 12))
 (segment (start 102.6084 88.3317) (end 102.5852 88.3549) (width 0.08) (layer F.Cu) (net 12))
 (segment (start 102.5852 88.3549) (end 102.3031 88.3549) (width 0.08) (layer F.Cu) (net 12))
 (segment (start 102.3031 88.3549) (end 102.108 88.55) (width 0.08) (layer F.Cu) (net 12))
 (via (at 103.3203 87.7694) (size 0.4) (drill 0.3) (layers F.Cu B.Cu) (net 12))
 (via (at 112.1359 100.33) (size 0.4) (drill 0.3) (layers F.Cu B.Cu) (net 12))
 (segment (start 102.808 88.55) (end 103.0374 88.3206) (width 0.08) (layer F.Cu) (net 13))
 (segment (start 103.0374 88.3206) (end 119.2846 88.3206) (width 0.08) (layer F.Cu) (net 13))
 (segment (start 119.2846 88.3206) (end 119.61 88.646) (width 0.08) (layer F.Cu) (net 13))
 (segment (start 120.65 88.646) (end 119.61 88.646) (width 0.08) (layer F.Cu) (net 13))
 (segment (start 93.4233 96.52) (end 91.582 96.52) (width 0.08) (layer F.Cu) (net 3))
 (segment (start 94.2085 96.5455) (end 93.4488 96.5455) (width 0.08) (layer F.Cu) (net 3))
 (segment (start 93.4488 96.5455) (end 93.4233 96.52) (width 0.08) (layer F.Cu) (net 3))
 (segment (start 102.108 89.95) (end 101.8568 90.2012) (width 0.08) (layer F.Cu) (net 3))
 (segment (start 101.8568 90.2012) (end 93.8702 90.2012) (width 0.08) (layer F.Cu) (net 3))
 (segment (start 93.8702 90.2012) (end 93.4233 90.6481) (width 0.08) (layer F.Cu) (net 3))
 (segment (start 93.4233 90.6481) (end 93.4233 96.52) (width 0.08) (layer F.Cu) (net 3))
 (segment (start 111.75 86.1164) (end 111.75 87.376) (width 1) (layer F.Cu) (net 4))
 (segment (start 112.5 86.106) (end 111.7604 86.106) (width 1) (layer F.Cu) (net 4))
 (segment (start 111.7604 86.106) (end 111.75 86.1164) (width 1) (layer F.Cu) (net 4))
 (segment (start 110.236 86.106) (end 111.7396 86.106) (width 1) (layer F.Cu) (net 4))
 (segment (start 111.7396 86.106) (end 111.75 86.1164) (width 1) (layer F.Cu) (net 4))
 (segment (start 97.025 86.106) (end 110.236 86.106) (width 1) (layer F.Cu) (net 4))
 (segment (start 113.25 87.376) (end 111.75 87.376) (width 1) (layer F.Cu) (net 4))
 (segment (start 113.25 86.106) (end 112.5 86.106) (width 1) (layer F.Cu) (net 4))
 (segment (start 97.025 86.106) (end 92.037 91.094) (width 1) (layer F.Cu) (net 4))
 (segment (start 92.037 91.094) (end 92.037 92.202) (width 1) (layer F.Cu) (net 4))
 (segment (start 97.025 86.106) (end 97.025 86.103) (width 1) (layer F.Cu) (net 4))
 (segment (start 97.025 86.103) (end 89.154 78.232) (width 1) (layer F.Cu) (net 4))
 (segment (start 89.662 92.202) (end 92.037 92.202) (width 1) (layer F.Cu) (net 4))
 (segment (start 89.662 92.202) (end 89.662 94.577) (width 1) (layer F.Cu) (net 4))
 (segment (start 89.662 94.577) (end 90.282 95.197) (width 1) (layer F.Cu) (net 4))
 (segment (start 90.282 95.197) (end 90.282 96.52) (width 1) (layer F.Cu) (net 4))
 (segment (start 112.5 97.79) (end 111.75 97.79) (width 1) (layer F.Cu) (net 4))
 (segment (start 113.25 97.79) (end 112.5 97.79) (width 1) (layer F.Cu) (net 4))
 (segment (start 112.5 99.06) (end 111.75 99.06) (width 1) (layer F.Cu) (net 4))
 (segment (start 113.25 99.06) (end 112.5 99.06) (width 1) (layer F.Cu) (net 4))
 (segment (start 112.5 97.79) (end 112.5 99.06) (width 1) (layer F.Cu) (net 4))
 (segment (start 110.2865 100.9582) (end 114.7637 105.4354) (width 1) (layer F.Cu) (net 4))
 (segment (start 114.7637 105.4354) (end 118.2876 105.4354) (width 1) (layer F.Cu) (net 4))
 (segment (start 118.2876 105.4354) (end 119.0899 104.6331) (width 1) (layer F.Cu) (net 4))
 (segment (start 119.0899 104.6331) (end 119.0899 99.805) (width 1) (layer F.Cu) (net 4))
 (segment (start 119.0899 99.805) (end 119.8349 99.06) (width 1) (layer F.Cu) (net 4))
 (segment (start 119.8349 99.06) (end 120.65 99.06) (width 1) (layer F.Cu) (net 4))
 (segment (start 104.3695 104.394) (end 107.8053 100.9582) (width 1) (layer F.Cu) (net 4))
 (segment (start 107.8053 100.9582) (end 110.2865 100.9582) (width 1) (layer F.Cu) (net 4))
 (segment (start 110.2865 100.9582) (end 111.75 99.4947) (width 1) (layer F.Cu) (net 4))
 (segment (start 111.75 99.4947) (end 111.75 99.06) (width 1) (layer F.Cu) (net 4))
 (segment (start 109.982 97.79) (end 111.75 97.79) (width 1) (layer F.Cu) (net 4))
 (segment (start 92.037 92.202) (end 92.037 92.7425) (width 1) (layer B.Cu) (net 4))
 (segment (start 92.037 92.7425) (end 102.2135 102.919) (width 1) (layer B.Cu) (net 4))
 (segment (start 102.2135 102.919) (end 103.632 102.919) (width 1) (layer B.Cu) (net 4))
 (segment (start 113.25 87.376) (end 120.65 87.376) (width 1) (layer F.Cu) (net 4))
 (segment (start 103.632 104.394) (end 103.632 102.919) (width 1) (layer B.Cu) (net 4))
 (segment (start 89.662 92.202) (end 92.037 92.202) (width 1) (layer B.Cu) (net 4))
 (segment (start 103.632 104.394) (end 104.3695 104.394) (width 1) (layer F.Cu) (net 4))
 (segment (start 110.966 81.5529) (end 110.966 80.232) (width 1) (layer B.Cu) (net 2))
 (segment (start 127.662 92.202) (end 120.5225 92.202) (width 1) (layer B.Cu) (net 2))
 (segment (start 120.5225 92.202) (end 110.966 82.6455) (width 1) (layer B.Cu) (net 2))
 (segment (start 110.966 82.6455) (end 110.966 81.5529) (width 1) (layer B.Cu) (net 2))
 (segment (start 110.966 81.5529) (end 107.4119 81.5529) (width 1) (layer B.Cu) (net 2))
 (segment (start 107.4119 81.5529) (end 105.615 79.756) (width 1) (layer B.Cu) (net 2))
 (segment (start 104.14 79.756) (end 105.615 79.756) (width 1) (layer B.Cu) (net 2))
 (segment (start 109.982 96.215) (end 105.8691 96.215) (width 1) (layer F.Cu) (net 2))
 (segment (start 105.8691 96.215) (end 102.1335 99.9506) (width 1) (layer F.Cu) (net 2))
 (segment (start 110.7973 95.3997) (end 109.982 96.215) (width 1) (layer F.Cu) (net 2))
 (segment (start 102.1335 99.9506) (end 102.1335 100.33) (width 1) (layer F.Cu) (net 2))
 (segment (start 94.234 94.945) (end 97.1279 94.945) (width 1) (layer F.Cu) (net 2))
 (segment (start 97.1279 94.945) (end 102.1335 99.9506) (width 1) (layer F.Cu) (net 2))
 (segment (start 94.234 94.945) (end 94.234 92.456) (width 1) (layer F.Cu) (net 2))
 (segment (start 94.2085 94.9705) (end 94.234 94.945) (width 1) (layer F.Cu) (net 2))
 (segment (start 120.65 96.52) (end 122.15 96.52) (width 1) (layer F.Cu) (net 2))
 (segment (start 127.662 92.202) (end 126.468 92.202) (width 1) (layer F.Cu) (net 2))
 (segment (start 126.468 92.202) (end 122.15 96.52) (width 1) (layer F.Cu) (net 2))
 (segment (start 110.966 80.232) (end 110.966 78.232) (width 1) (layer B.Cu) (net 2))
 (segment (start 119.15 96.52) (end 118.0297 95.3997) (width 1) (layer F.Cu) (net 2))
 (segment (start 118.0297 95.3997) (end 110.7973 95.3997) (width 1) (layer F.Cu) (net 2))
 (segment (start 110.7973 95.3997) (end 110.7973 90.9853) (width 1) (layer F.Cu) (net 2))
 (segment (start 110.7973 90.9853) (end 109.982 90.17) (width 1) (layer F.Cu) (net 2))
 (segment (start 91.694 78.232) (end 91.694 79.857) (width 1) (layer B.Cu) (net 2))
 (segment (start 91.694 79.857) (end 95.4673 79.857) (width 1) (layer B.Cu) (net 2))
 (segment (start 95.4673 79.857) (end 97.0395 78.2848) (width 1) (layer B.Cu) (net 2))
 (segment (start 97.0395 78.2848) (end 102.6688 78.2848) (width 1) (layer B.Cu) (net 2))
 (segment (start 102.6688 78.2848) (end 104.14 79.756) (width 1) (layer B.Cu) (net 2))
 (segment (start 110.966 83.3814) (end 117.6954 83.3814) (width 1) (layer F.Cu) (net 2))
 (segment (start 117.6954 83.3814) (end 119.15 84.836) (width 1) (layer F.Cu) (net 2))
 (segment (start 110.236 84.531) (end 110.236 84.1114) (width 1) (layer F.Cu) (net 2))
 (segment (start 110.236 84.1114) (end 110.966 83.3814) (width 1) (layer F.Cu) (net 2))
 (segment (start 110.966 83.3814) (end 110.966 81.532) (width 1) (layer F.Cu) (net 2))
 (segment (start 120.65 84.836) (end 119.15 84.836) (width 1) (layer F.Cu) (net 2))
 (segment (start 101.092 104.394) (end 101.092 102.919) (width 1) (layer F.Cu) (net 2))
 (segment (start 102.1335 100.33) (end 102.1335 101.8775) (width 1) (layer F.Cu) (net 2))
 (segment (start 102.1335 101.8775) (end 101.092 102.919) (width 1) (layer F.Cu) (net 2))
 (segment (start 110.966 80.232) (end 110.966 81.532) (width 1) (layer F.Cu) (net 2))
 (segment (start 120.65 96.52) (end 119.15 96.52) (width 1) (layer F.Cu) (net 2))
 (segment (start 102.458 89.95) (end 102.6175 89.7905) (width 0.08) (layer F.Cu) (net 1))
 (segment (start 102.6175 89.7905) (end 102.6175 89.5209) (width 0.08) (layer F.Cu) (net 1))
 (segment (start 102.6175 89.5209) (end 102.7334 89.405) (width 0.08) (layer F.Cu) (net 1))
 (segment (start 102.7334 89.405) (end 107.917 89.405) (width 0.08) (layer F.Cu) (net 1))
 (segment (start 107.917 89.405) (end 108.682 90.17) (width 0.08) (layer F.Cu) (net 1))
 (segment (start 100.3267 88.9223) (end 101.3857 88.9223) (width 0.25) (layer F.Cu) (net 9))
 (segment (start 101.3857 88.9223) (end 101.408 88.9) (width 0.25) (layer F.Cu) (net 9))
 (segment (start 97.6156 96.8783) (end 97.6156 91.6334) (width 0.25) (layer B.Cu) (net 9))
 (segment (start 97.6156 91.6334) (end 100.3267 88.9223) (width 0.25) (layer B.Cu) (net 9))
 (segment (start 97.056 100.33) (end 97.6156 99.7704) (width 0.25) (layer F.Cu) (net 9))
 (segment (start 97.6156 99.7704) (end 97.6156 96.8783) (width 0.25) (layer F.Cu) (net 9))
 (via (at 100.3267 88.9223) (size 0.8) (layers F.Cu B.Cu) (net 9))
 (via (at 97.6156 96.8783) (size 0.8) (layers F.Cu B.Cu) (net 9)))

